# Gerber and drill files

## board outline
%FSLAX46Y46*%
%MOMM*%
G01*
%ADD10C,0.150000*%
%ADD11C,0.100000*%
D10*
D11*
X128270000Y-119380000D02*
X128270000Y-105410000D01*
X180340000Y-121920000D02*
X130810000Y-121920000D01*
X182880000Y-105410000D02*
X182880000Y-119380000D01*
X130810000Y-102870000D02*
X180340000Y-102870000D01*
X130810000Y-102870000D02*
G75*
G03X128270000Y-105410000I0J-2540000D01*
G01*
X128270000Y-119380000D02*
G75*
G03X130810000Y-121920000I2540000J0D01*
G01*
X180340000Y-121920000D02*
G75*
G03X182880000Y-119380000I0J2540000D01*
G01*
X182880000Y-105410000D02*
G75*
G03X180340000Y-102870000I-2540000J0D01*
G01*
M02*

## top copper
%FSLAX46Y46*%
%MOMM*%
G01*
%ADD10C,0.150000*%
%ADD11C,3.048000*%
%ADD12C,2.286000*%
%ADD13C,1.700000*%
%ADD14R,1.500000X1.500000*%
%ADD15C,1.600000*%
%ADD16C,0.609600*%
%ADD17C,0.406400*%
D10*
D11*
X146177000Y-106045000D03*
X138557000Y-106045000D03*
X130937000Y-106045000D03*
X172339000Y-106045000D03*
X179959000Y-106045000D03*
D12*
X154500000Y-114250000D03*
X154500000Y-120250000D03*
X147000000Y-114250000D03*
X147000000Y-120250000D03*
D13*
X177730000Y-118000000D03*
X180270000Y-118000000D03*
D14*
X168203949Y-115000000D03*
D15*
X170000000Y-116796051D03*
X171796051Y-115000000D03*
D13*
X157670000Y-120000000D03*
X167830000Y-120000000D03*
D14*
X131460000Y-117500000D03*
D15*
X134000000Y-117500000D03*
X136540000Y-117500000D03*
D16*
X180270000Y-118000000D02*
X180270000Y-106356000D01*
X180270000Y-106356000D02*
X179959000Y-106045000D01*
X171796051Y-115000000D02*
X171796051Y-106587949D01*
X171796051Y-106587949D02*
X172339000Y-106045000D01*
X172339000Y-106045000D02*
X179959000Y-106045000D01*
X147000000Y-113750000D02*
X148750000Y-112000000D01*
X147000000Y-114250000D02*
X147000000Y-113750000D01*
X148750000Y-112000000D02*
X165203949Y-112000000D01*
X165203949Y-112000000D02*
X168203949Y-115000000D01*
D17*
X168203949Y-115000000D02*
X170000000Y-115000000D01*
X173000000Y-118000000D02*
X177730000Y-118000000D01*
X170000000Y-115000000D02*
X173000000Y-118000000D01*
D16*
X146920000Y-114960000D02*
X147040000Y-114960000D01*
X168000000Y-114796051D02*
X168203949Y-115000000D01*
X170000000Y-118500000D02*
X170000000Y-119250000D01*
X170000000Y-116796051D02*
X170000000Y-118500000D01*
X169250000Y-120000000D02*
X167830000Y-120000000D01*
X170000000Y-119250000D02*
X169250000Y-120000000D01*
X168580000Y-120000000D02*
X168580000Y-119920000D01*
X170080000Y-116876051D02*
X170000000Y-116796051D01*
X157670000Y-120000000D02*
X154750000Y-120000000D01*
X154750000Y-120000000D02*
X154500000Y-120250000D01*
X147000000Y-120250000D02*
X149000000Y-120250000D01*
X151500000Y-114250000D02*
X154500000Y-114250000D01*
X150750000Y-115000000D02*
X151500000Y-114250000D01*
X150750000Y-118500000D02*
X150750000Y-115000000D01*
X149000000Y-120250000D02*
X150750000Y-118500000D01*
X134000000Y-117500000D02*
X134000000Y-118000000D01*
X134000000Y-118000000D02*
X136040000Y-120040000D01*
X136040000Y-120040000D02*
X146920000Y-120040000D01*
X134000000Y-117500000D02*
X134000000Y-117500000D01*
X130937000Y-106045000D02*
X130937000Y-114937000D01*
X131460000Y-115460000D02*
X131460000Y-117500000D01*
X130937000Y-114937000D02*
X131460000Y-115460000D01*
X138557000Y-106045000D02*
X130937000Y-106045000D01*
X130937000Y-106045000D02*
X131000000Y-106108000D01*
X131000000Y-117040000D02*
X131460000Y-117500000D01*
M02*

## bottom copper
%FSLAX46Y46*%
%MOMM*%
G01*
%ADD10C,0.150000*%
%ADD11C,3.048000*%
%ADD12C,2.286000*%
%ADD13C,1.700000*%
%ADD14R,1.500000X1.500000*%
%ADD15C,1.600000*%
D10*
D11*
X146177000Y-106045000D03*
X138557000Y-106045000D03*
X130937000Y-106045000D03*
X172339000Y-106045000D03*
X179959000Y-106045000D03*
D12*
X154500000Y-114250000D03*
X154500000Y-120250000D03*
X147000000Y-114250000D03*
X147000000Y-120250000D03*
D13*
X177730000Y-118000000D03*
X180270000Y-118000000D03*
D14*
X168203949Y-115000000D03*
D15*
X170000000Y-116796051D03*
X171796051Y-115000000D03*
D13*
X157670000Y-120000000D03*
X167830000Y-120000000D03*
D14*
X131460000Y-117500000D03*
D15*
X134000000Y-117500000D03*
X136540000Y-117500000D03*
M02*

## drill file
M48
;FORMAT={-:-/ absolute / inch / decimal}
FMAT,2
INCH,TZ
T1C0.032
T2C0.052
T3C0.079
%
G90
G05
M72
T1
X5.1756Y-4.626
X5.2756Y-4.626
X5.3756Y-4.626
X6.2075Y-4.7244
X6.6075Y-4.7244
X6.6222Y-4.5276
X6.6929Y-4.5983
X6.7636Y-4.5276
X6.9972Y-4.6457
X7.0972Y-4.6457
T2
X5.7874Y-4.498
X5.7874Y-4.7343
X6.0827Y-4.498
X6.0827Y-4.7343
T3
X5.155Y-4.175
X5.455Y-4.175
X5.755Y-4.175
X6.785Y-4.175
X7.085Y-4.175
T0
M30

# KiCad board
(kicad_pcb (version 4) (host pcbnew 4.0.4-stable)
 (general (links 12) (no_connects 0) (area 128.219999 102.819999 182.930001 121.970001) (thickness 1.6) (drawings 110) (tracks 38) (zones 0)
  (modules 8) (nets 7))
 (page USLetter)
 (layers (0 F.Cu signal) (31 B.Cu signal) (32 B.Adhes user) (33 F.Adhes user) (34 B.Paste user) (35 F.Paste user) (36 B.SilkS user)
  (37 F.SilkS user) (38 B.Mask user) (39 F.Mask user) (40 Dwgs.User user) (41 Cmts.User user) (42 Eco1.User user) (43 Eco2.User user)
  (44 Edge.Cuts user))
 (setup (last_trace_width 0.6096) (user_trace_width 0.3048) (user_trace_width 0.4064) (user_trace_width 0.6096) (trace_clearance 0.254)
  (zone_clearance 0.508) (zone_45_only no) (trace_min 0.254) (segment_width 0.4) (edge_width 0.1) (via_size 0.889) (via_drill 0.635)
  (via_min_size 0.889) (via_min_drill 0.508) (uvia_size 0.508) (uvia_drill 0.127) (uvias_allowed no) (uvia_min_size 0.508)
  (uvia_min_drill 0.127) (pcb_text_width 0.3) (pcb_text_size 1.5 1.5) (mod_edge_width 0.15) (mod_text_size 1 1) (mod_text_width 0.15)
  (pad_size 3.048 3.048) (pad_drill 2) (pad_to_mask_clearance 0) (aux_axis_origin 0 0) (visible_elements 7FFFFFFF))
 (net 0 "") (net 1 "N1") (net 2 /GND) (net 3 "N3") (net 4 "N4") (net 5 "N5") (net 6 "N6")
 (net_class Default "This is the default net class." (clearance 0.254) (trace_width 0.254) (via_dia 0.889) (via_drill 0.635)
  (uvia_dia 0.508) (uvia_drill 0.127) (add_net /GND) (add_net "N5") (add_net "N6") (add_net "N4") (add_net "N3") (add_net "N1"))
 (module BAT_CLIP (layer F.Cu) (at 155.575 106.045)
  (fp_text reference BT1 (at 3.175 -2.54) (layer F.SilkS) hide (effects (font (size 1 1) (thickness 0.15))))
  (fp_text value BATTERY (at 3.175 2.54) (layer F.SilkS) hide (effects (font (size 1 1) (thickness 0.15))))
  (pad 1 thru_hole circle (at -9.398 0) (size 3.048 3.048) (drill 2) (layers *.Cu *.Mask) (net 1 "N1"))
  (pad 1 thru_hole circle (at -17.018 0) (size 3.048 3.048) (drill 2) (layers *.Cu *.Mask) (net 1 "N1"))
  (pad 1 thru_hole circle (at -24.638 0) (size 3.048 3.048) (drill 2) (layers *.Cu *.Mask) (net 1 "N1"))
  (pad 2 thru_hole circle (at 16.764 0) (size 3.048 3.048) (drill 2) (layers *.Cu *.Mask) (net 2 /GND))
  (pad 2 thru_hole circle (at 24.384 0) (size 3.048 3.048) (drill 2) (layers *.Cu *.Mask) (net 2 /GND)))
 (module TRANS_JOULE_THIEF (layer F.Cu) (at 152 117.25 270)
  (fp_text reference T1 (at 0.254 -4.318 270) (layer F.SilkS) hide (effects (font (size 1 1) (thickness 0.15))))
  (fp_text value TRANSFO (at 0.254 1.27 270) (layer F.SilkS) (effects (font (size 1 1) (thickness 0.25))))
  (pad 1 thru_hole circle (at -3 -2.5 270) (size 2.286 2.286) (drill 1.3208) (layers *.Cu B.Mask) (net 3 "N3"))
  (pad 2 thru_hole circle (at 3 -2.5 270) (size 2.286 2.286) (drill 1.3208) (layers *.Cu B.Mask) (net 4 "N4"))
  (pad 3 thru_hole circle (at -3 5 270) (size 2.286 2.286) (drill 1.3208) (layers *.Cu B.Mask) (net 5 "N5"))
  (pad 4 thru_hole circle (at 3 5 270) (size 2.286 2.286) (drill 1.3208) (layers *.Cu B.Mask) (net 3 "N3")))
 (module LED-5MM (layer F.Cu) (at 179 118)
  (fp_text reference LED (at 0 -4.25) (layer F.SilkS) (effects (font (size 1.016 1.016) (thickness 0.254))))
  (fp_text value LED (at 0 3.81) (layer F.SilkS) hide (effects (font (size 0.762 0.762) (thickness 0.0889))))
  (pad 1 thru_hole circle (at -1.27 0) (size 1.7 1.7) (drill 0.8128) (layers *.Cu B.Mask) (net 5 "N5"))
  (pad 2 thru_hole circle (at 1.27 0) (size 1.7 1.7) (drill 0.8128) (layers *.Cu B.Mask) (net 2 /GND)))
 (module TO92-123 (layer F.Cu) (at 170 115 135)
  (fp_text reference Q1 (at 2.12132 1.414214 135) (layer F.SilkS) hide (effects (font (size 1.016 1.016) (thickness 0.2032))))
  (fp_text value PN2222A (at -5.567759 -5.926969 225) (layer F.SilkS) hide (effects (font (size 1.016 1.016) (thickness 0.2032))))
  (pad 3 thru_hole rect (at 1.27 -1.27 180) (size 1.5 1.5) (drill 0.8128) (layers *.Cu B.Mask) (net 5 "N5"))
  (pad 2 thru_hole circle (at -1.27 -1.27 135) (size 1.6 1.6) (drill 0.8128) (layers *.Cu B.Mask) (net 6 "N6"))
  (pad 1 thru_hole circle (at -1.27 1.27 135) (size 1.6 1.6) (drill 0.8128) (layers *.Cu B.Mask) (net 2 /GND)))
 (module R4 (layer F.Cu) (at 162.75 120) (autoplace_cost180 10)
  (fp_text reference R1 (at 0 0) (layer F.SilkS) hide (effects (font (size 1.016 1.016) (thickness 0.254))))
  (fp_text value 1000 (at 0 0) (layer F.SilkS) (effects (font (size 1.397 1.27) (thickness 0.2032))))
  (pad 1 thru_hole circle (at -5.08 0) (size 1.7 1.7) (drill 0.8128) (layers *.Cu B.Mask) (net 4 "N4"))
  (pad 2 thru_hole circle (at 5.08 0) (size 1.7 1.7) (drill 0.8128) (layers *.Cu B.Mask) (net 6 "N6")))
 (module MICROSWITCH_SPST (layer F.Cu) (at 134 117.5)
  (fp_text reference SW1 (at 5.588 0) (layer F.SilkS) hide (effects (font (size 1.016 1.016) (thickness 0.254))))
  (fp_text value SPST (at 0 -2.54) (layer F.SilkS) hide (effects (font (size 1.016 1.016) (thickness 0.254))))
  (pad 1 thru_hole rect (at -2.54 0) (size 1.5 1.5) (drill 0.8128) (layers *.Cu B.Mask) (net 1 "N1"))
  (pad 2 thru_hole circle (at 0 0) (size 1.6 1.6) (drill 0.8128) (layers *.Cu B.Mask) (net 3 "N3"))
  (pad 3 thru_hole circle (at 2.54 0) (size 1.6 1.6) (drill 0.8128) (layers *.Cu B.Mask)))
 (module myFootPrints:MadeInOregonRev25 (layer F.Cu) (at 134 111.5)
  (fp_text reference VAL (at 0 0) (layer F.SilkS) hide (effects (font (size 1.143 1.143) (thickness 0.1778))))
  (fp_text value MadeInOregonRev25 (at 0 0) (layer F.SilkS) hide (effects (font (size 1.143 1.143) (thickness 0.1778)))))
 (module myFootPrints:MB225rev (layer F.Cu) (at 141 111.5)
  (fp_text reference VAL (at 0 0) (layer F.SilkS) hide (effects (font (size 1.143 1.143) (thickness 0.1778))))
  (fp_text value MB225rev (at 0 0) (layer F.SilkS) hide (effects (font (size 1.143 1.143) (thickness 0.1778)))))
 (gr_line (start 128.27 119.38) (end 128.27 105.41) (angle 90) (layer Edge.Cuts) (width 0.1))
 (gr_line (start 180.34 121.92) (end 130.81 121.92) (angle 90) (layer Edge.Cuts) (width 0.1))
 (gr_line (start 182.88 105.41) (end 182.88 119.38) (angle 90) (layer Edge.Cuts) (width 0.1))
 (gr_line (start 130.81 102.87) (end 180.34 102.87) (angle 90) (layer Edge.Cuts) (width 0.1))
 (gr_arc (start 130.81 105.41) (end 128.27 105.41) (angle 90) (layer Edge.Cuts) (width 0.1))
 (gr_arc (start 130.81 119.38) (end 130.81 121.92) (angle 90) (layer Edge.Cuts) (width 0.1))
 (gr_arc (start 180.34 119.38) (end 182.88 119.38) (angle 90) (layer Edge.Cuts) (width 0.1))
 (gr_arc (start 180.34 105.41) (end 180.34 102.87) (angle 90) (layer Edge.Cuts) (width 0.1))
 (segment (start 180.27 118) (end 180.27 106.356) (width 0.6096) (layer F.Cu) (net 2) (status 10))
 (segment (start 180.27 106.356) (end 179.959 106.045) (width 0.6096) (layer F.Cu) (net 2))
 (segment (start 171.796051 115) (end 171.796051 106.587949) (width 0.6096) (layer F.Cu) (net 2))
 (segment (start 171.796051 106.587949) (end 172.339 106.045) (width 0.6096) (layer F.Cu) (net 2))
 (segment (start 172.339 106.045) (end 179.959 106.045) (width 0.6096) (layer F.Cu) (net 2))
 (segment (start 147 113.75) (end 148.75 112) (width 0.6096) (layer F.Cu) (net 5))
 (segment (start 147 114.25) (end 147 113.75) (width 0.6096) (layer F.Cu) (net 5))
 (segment (start 148.75 112) (end 165.203949 112) (width 0.6096) (layer F.Cu) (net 5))
 (segment (start 165.203949 112) (end 168.203949 115) (width 0.6096) (layer F.Cu) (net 5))
 (segment (start 168.203949 115) (end 170 115) (width 0.4064) (layer F.Cu) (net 5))
 (segment (start 173 118) (end 177.73 118) (width 0.4064) (layer F.Cu) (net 5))
 (segment (start 170 115) (end 173 118) (width 0.4064) (layer F.Cu) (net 5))
 (segment (start 146.92 114.96) (end 147.04 114.96) (width 0.6096) (layer F.Cu) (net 5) (status 30))
 (segment (start 168 114.796051) (end 168.203949 115) (width 0.6096) (layer F.Cu) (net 5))
 (segment (start 170 118.5) (end 170 119.25) (width 0.6096) (layer F.Cu) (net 6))
 (segment (start 170 116.796051) (end 170 118.5) (width 0.6096) (layer F.Cu) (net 6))
 (segment (start 169.25 120) (end 167.83 120) (width 0.6096) (layer F.Cu) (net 6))
 (segment (start 170 119.25) (end 169.25 120) (width 0.6096) (layer F.Cu) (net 6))
 (segment (start 168.58 120) (end 168.58 119.92) (width 0.6096) (layer F.Cu) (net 6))
 (segment (start 170.08 116.876051) (end 170 116.796051) (width 0.6096) (layer F.Cu) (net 6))
 (segment (start 157.67 120) (end 154.75 120) (width 0.6096) (layer F.Cu) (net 4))
 (segment (start 154.75 120) (end 154.5 120.25) (width 0.6096) (layer F.Cu) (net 4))
 (segment (start 147 120.25) (end 149 120.25) (width 0.6096) (layer F.Cu) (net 3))
 (segment (start 151.5 114.25) (end 154.5 114.25) (width 0.6096) (layer F.Cu) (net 3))
 (segment (start 150.75 115) (end 151.5 114.25) (width 0.6096) (layer F.Cu) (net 3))
 (segment (start 150.75 118.5) (end 150.75 115) (width 0.6096) (layer F.Cu) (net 3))
 (segment (start 149 120.25) (end 150.75 118.5) (width 0.6096) (layer F.Cu) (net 3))
 (segment (start 134 117.5) (end 134 118) (width 0.6096) (layer F.Cu) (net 3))
 (segment (start 134 118) (end 136.04 120.04) (width 0.6096) (layer F.Cu) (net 3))
 (segment (start 136.04 120.04) (end 146.92 120.04) (width 0.6096) (layer F.Cu) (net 3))
 (segment (start 134 117.5) (end 134 117.5) (width 0.6096) (layer F.Cu) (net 3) (status 10))
 (segment (start 138.557 106.045) (end 146.177 106.045) (width 0.6096) (layer F.Cu) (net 1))
 (segment (start 130.937 106.045) (end 130.937 114.937) (width 0.6096) (layer F.Cu) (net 1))
 (segment (start 131.46 115.46) (end 131.46 117.5) (width 0.6096) (layer F.Cu) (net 1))
 (segment (start 130.937 114.937) (end 131.46 115.46) (width 0.6096) (layer F.Cu) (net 1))
 (segment (start 138.557 106.045) (end 130.937 106.045) (width 0.6096) (layer F.Cu) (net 1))
 (segment (start 130.937 106.045) (end 131 106.108) (width 0.6096) (layer F.Cu) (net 1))
 (segment (start 131 117.04) (end 131.46 117.5) (width 0.6096) (layer F.Cu) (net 1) (status 30)))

